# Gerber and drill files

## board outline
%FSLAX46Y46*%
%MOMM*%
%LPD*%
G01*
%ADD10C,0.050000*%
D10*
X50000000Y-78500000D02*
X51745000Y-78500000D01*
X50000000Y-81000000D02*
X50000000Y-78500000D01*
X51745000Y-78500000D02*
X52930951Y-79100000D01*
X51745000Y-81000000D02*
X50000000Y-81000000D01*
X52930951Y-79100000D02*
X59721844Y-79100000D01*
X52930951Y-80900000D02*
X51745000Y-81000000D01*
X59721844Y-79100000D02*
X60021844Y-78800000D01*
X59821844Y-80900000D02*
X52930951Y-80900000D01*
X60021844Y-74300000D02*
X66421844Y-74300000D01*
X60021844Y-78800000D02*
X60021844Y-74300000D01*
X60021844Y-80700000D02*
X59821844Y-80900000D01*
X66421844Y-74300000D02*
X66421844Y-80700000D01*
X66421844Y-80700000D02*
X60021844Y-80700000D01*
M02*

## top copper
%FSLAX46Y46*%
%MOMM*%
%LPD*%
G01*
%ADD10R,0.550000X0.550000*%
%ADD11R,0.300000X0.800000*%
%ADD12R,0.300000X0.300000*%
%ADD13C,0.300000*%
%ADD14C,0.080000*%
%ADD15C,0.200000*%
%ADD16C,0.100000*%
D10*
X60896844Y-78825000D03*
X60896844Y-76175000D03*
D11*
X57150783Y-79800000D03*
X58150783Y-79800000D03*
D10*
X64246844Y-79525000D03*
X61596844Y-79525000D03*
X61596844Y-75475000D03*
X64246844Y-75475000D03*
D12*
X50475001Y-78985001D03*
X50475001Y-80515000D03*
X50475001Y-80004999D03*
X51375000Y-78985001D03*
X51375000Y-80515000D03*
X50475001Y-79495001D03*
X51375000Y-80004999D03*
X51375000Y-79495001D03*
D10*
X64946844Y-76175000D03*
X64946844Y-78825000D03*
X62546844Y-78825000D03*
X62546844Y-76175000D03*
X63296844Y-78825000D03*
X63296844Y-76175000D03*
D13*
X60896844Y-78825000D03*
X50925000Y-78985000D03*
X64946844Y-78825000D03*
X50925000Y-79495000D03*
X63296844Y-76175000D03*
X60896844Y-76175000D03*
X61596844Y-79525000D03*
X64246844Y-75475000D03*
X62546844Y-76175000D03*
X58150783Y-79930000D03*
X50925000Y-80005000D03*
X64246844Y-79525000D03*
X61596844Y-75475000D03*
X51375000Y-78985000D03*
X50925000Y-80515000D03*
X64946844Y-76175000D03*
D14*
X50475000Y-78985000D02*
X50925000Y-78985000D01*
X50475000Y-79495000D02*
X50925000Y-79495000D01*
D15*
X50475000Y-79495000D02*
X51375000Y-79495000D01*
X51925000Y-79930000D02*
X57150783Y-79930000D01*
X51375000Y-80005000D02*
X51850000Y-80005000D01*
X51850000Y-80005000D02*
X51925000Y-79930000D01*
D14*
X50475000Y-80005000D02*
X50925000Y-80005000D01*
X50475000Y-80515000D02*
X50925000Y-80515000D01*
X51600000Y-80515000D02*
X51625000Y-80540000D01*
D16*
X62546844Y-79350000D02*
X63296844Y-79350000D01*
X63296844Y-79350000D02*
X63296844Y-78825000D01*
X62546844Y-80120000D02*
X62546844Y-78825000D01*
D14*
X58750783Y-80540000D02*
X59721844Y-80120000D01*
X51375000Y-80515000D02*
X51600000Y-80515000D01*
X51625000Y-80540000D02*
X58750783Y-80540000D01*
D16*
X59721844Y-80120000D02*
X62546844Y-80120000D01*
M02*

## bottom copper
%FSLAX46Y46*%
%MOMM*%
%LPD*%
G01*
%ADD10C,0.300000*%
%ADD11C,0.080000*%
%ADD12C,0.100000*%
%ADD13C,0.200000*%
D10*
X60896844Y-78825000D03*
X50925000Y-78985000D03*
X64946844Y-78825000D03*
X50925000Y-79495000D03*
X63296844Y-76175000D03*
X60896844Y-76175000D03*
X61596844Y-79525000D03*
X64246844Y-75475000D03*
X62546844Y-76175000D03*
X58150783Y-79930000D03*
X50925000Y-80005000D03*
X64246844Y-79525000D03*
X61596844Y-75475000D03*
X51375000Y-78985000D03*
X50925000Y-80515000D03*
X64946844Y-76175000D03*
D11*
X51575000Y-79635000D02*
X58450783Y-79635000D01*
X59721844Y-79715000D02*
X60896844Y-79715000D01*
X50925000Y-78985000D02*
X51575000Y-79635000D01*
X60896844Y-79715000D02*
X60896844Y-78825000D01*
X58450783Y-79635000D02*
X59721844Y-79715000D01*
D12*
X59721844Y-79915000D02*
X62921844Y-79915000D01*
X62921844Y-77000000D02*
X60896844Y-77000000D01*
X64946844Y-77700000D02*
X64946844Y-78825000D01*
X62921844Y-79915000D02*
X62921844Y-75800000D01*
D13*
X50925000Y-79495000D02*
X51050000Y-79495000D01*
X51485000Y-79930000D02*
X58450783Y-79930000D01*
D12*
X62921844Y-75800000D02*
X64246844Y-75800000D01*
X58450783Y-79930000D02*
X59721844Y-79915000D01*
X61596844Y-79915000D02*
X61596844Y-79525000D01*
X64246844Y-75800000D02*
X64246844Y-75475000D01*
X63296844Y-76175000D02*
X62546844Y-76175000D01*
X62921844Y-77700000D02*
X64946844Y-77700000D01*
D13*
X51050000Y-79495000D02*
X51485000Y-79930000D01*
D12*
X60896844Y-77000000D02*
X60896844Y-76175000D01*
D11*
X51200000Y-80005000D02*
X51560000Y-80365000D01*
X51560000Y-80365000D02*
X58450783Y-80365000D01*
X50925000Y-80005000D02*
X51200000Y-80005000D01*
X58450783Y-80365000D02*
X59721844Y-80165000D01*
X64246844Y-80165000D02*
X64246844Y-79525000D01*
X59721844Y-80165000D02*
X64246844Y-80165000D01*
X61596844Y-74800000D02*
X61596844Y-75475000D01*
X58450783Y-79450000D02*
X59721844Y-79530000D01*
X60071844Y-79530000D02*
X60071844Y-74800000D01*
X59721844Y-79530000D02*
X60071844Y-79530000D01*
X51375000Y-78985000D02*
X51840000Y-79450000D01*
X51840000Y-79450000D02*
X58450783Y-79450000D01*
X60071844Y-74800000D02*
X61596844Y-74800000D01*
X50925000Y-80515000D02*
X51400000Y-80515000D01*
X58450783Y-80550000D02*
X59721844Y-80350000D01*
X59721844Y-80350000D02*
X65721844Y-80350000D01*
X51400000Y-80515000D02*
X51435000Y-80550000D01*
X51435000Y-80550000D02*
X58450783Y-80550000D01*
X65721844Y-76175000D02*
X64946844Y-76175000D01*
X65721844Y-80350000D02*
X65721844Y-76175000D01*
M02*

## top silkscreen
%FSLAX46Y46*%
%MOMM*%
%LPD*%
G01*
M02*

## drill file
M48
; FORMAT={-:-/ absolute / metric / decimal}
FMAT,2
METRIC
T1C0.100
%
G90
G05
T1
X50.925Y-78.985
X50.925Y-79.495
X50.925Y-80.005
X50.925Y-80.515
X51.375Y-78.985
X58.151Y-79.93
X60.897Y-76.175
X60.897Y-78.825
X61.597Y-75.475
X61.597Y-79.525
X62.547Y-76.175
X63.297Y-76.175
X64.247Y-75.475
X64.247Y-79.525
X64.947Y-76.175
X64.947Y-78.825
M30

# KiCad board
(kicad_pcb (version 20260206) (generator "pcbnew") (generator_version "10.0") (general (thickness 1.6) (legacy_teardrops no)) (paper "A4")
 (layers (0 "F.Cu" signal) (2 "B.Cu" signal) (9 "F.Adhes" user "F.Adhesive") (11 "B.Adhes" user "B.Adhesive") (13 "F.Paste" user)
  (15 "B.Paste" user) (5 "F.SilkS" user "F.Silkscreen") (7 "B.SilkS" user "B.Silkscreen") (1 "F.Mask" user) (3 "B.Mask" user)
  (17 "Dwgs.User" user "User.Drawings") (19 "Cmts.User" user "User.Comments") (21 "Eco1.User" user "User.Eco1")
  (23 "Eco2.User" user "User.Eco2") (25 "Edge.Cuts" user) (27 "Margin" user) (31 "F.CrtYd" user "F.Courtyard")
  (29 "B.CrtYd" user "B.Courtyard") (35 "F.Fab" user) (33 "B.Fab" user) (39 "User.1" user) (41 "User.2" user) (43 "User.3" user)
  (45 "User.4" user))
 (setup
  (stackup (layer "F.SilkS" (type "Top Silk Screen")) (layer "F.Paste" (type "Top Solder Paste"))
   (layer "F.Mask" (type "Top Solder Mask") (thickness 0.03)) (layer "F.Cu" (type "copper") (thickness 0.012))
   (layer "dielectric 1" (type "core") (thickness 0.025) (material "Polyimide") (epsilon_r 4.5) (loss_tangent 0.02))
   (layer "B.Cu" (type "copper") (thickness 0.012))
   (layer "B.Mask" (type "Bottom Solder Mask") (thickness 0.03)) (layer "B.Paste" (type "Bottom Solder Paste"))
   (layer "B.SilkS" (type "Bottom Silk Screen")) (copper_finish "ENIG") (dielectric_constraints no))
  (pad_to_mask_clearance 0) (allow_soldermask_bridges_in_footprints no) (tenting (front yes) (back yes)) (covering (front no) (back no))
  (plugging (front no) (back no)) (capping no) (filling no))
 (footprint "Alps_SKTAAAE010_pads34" (layer "F.Cu") (at 60.521844 77.5 90)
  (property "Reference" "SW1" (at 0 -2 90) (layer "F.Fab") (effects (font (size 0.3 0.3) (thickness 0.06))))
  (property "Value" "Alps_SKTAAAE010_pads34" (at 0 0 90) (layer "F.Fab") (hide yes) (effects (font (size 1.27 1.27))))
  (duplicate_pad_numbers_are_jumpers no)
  (pad "3" smd rect (at -1.325 0.375 90) (size 0.55 0.55) (layers "F.Cu" "F.Mask") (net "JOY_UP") (solder_mask_margin 0.05)
   (thermal_bridge_angle 45))
  (pad "4" smd rect (at 1.325 0.375 90) (size 0.55 0.55) (layers "F.Cu" "F.Mask") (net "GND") (solder_mask_margin 0.05)
   (thermal_bridge_angle 45)))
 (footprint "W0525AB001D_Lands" (layer "F.Cu") (at 57.650783 79.93)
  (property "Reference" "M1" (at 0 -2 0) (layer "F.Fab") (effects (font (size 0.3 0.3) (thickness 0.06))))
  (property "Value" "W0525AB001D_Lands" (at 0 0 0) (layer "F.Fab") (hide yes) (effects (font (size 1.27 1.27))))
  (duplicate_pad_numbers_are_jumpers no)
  (pad "1" smd rect (at -0.5 -0.13) (size 0.3 0.8) (layers "F.Cu" "F.Mask") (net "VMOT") (solder_mask_margin 0.05) (thermal_bridge_angle 45))
  (pad "2" smd rect (at 0.5 -0.13) (size 0.3 0.8) (layers "F.Cu" "F.Mask") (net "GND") (solder_mask_margin 0.05) (thermal_bridge_angle 45)))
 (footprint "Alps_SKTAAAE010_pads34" (layer "F.Cu") (at 62.921844 79.9 180)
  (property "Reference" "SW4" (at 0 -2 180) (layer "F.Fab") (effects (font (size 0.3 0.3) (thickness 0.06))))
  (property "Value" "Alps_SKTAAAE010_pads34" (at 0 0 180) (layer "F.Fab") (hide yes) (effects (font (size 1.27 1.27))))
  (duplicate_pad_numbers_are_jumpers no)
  (pad "3" smd rect (at -1.325 0.375 180) (size 0.55 0.55) (layers "F.Cu" "F.Mask") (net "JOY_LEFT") (solder_mask_margin 0.05)
   (thermal_bridge_angle 45))
  (pad "4" smd rect (at 1.325 0.375 180) (size 0.55 0.55) (layers "F.Cu" "F.Mask") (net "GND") (solder_mask_margin 0.05)
   (thermal_bridge_angle 45)))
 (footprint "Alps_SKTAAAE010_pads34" (layer "F.Cu") (at 62.921844 75.1)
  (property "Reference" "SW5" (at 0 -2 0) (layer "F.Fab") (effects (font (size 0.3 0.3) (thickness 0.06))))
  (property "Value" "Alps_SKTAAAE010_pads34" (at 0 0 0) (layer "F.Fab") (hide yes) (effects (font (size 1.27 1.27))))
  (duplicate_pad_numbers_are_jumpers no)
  (pad "3" smd rect (at -1.325 0.375) (size 0.55 0.55) (layers "F.Cu" "F.Mask") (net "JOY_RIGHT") (solder_mask_margin 0.05)
   (thermal_bridge_angle 45))
  (pad "4" smd rect (at 1.325 0.375) (size 0.55 0.55) (layers "F.Cu" "F.Mask") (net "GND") (solder_mask_margin 0.05)
   (thermal_bridge_angle 45)))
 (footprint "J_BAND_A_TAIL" (layer "F.Cu") (at 50.9 79.75)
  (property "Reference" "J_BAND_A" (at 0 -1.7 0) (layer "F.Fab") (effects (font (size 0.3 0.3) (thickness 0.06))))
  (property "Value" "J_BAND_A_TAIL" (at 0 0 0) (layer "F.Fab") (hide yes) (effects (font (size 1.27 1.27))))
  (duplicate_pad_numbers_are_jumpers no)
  (pad "1" smd rect (at -0.424999 -0.764999) (size 0.3 0.3) (layers "F.Cu" "F.Mask") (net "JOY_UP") (solder_mask_margin 0.05)
   (thermal_bridge_angle 45))
  (pad "2" smd rect (at -0.424999 0.765) (size 0.3 0.3) (layers "F.Cu" "F.Mask") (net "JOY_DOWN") (solder_mask_margin 0.05)
   (thermal_bridge_angle 45))
  (pad "3" smd rect (at -0.424999 0.254999) (size 0.3 0.3) (layers "F.Cu" "F.Mask") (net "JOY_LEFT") (solder_mask_margin 0.05)
   (thermal_bridge_angle 45))
  (pad "4" smd rect (at 0.475 -0.764999) (size 0.3 0.3) (layers "F.Cu" "F.Mask") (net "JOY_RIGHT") (solder_mask_margin 0.05)
   (thermal_bridge_angle 45))
  (pad "5" smd rect (at 0.475 0.765) (size 0.3 0.3) (layers "F.Cu" "F.Mask") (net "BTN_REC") (solder_mask_margin 0.05)
   (thermal_bridge_angle 45))
  (pad "6" smd rect (at -0.424999 -0.254999) (size 0.3 0.3) (layers "F.Cu" "F.Mask") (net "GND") (solder_mask_margin 0.05)
   (thermal_bridge_angle 45))
  (pad "7" smd rect (at 0.475 0.254999) (size 0.3 0.3) (layers "F.Cu" "F.Mask") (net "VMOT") (solder_mask_margin 0.05)
   (thermal_bridge_angle 45))
  (pad "8" smd rect (at 0.475 -0.254999) (size 0.3 0.3) (layers "F.Cu" "F.Mask") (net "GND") (solder_mask_margin 0.05)
   (thermal_bridge_angle 45)))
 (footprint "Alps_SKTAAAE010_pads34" (layer "F.Cu") (at 65.321844 77.5 -90)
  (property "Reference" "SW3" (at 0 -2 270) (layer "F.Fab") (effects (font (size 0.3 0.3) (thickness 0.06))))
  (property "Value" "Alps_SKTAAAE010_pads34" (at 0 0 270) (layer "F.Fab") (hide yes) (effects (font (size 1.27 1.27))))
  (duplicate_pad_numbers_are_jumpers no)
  (pad "3" smd rect (at -1.325 0.375 270) (size 0.55 0.55) (layers "F.Cu" "F.Mask") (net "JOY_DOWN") (solder_mask_margin 0.05)
   (thermal_bridge_angle 45))
  (pad "4" smd rect (at 1.325 0.375 270) (size 0.55 0.55) (layers "F.Cu" "F.Mask") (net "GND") (solder_mask_margin 0.05)
   (thermal_bridge_angle 45)))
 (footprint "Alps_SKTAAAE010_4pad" (layer "F.Cu") (at 62.921844 77.5 90)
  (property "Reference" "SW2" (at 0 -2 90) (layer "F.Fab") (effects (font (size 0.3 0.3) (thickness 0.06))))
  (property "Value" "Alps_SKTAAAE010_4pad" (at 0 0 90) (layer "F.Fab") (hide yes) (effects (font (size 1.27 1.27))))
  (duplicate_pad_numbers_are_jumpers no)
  (pad "1" smd rect (at -1.325 -0.375 90) (size 0.55 0.55) (layers "F.Cu" "F.Mask") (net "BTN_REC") (solder_mask_margin 0.05)
   (thermal_bridge_angle 45))
  (pad "2" smd rect (at 1.325 -0.375 90) (size 0.55 0.55) (layers "F.Cu" "F.Mask") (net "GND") (solder_mask_margin 0.05)
   (thermal_bridge_angle 45))
  (pad "3" smd rect (at -1.325 0.375 90) (size 0.55 0.55) (layers "F.Cu" "F.Mask") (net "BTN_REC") (solder_mask_margin 0.05)
   (thermal_bridge_angle 45))
  (pad "4" smd rect (at 1.325 0.375 90) (size 0.55 0.55) (layers "F.Cu" "F.Mask") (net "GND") (solder_mask_margin 0.05)
   (thermal_bridge_angle 45)))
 (gr_line (start 50 78.5) (end 51.745 78.5) (stroke (width 0.05) (type default)) (layer "Edge.Cuts"))
 (gr_line (start 50 81) (end 50 78.5) (stroke (width 0.05) (type default)) (layer "Edge.Cuts"))
 (gr_line (start 51.745 78.5) (end 52.930951 79.1) (stroke (width 0.05) (type default)) (layer "Edge.Cuts"))
 (gr_line (start 51.745 81) (end 50 81) (stroke (width 0.05) (type default)) (layer "Edge.Cuts"))
 (gr_line (start 52.930951 79.1) (end 59.721844 79.1) (stroke (width 0.05) (type default)) (layer "Edge.Cuts"))
 (gr_line (start 52.930951 80.9) (end 51.745 81) (stroke (width 0.05) (type default)) (layer "Edge.Cuts"))
 (gr_line (start 59.721844 79.1) (end 60.021844 78.8) (stroke (width 0.05) (type default)) (layer "Edge.Cuts"))
 (gr_line (start 59.821844 80.9) (end 52.930951 80.9) (stroke (width 0.05) (type default)) (layer "Edge.Cuts"))
 (gr_line (start 60.021844 74.3) (end 66.421844 74.3) (stroke (width 0.05) (type default)) (layer "Edge.Cuts"))
 (gr_line (start 60.021844 78.8) (end 60.021844 74.3) (stroke (width 0.05) (type default)) (layer "Edge.Cuts"))
 (gr_line (start 60.021844 80.7) (end 59.821844 80.9) (stroke (width 0.05) (type default)) (layer "Edge.Cuts"))
 (gr_line (start 66.421844 74.3) (end 66.421844 80.7) (stroke (width 0.05) (type default)) (layer "Edge.Cuts"))
 (gr_line (start 66.421844 80.7) (end 60.021844 80.7) (stroke (width 0.05) (type default)) (layer "Edge.Cuts"))
 (segment (start 50.475 78.985) (end 50.925 78.985) (width 0.08) (layer "F.Cu") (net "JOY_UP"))
 (via (at 60.896844 78.825) (size 0.3) (drill 0.1) (layers "F.Cu" "B.Cu") (tenting (front yes) (back yes)) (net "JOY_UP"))
 (via (at 50.925 78.985) (size 0.3) (drill 0.1) (layers "F.Cu" "B.Cu") (tenting (front yes) (back yes)) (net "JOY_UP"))
 (segment (start 51.575 79.635) (end 58.450783 79.635) (width 0.08) (layer "B.Cu") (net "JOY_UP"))
 (segment (start 59.721844 79.715) (end 60.896844 79.715) (width 0.08) (layer "B.Cu") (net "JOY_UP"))
 (segment (start 50.925 78.985) (end 51.575 79.635) (width 0.08) (layer "B.Cu") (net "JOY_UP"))
 (segment (start 60.896844 79.715) (end 60.896844 78.825) (width 0.08) (layer "B.Cu") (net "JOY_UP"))
 (segment (start 58.450783 79.635) (end 59.721844 79.715) (width 0.08) (layer "B.Cu") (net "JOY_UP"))
 (segment (start 50.475 79.495) (end 50.925 79.495) (width 0.08) (layer "F.Cu") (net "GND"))
 (segment (start 50.475 79.495) (end 51.375 79.495) (width 0.2) (layer "F.Cu") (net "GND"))
 (via (at 64.946844 78.825) (size 0.3) (drill 0.1) (layers "F.Cu" "B.Cu") (tenting (front yes) (back yes)) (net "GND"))
 (via (at 50.925 79.495) (size 0.3) (drill 0.1) (layers "F.Cu" "B.Cu") (tenting (front yes) (back yes)) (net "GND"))
 (via (at 63.296844 76.175) (size 0.3) (drill 0.1) (layers "F.Cu" "B.Cu") (tenting (front yes) (back yes)) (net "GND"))
 (via (at 60.896844 76.175) (size 0.3) (drill 0.1) (layers "F.Cu" "B.Cu") (tenting (front yes) (back yes)) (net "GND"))
 (via (at 61.596844 79.525) (size 0.3) (drill 0.1) (layers "F.Cu" "B.Cu") (tenting (front yes) (back yes)) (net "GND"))
 (via (at 64.246844 75.475) (size 0.3) (drill 0.1) (layers "F.Cu" "B.Cu") (tenting (front yes) (back yes)) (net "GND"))
 (via (at 62.546844 76.175) (size 0.3) (drill 0.1) (layers "F.Cu" "B.Cu") (tenting (front yes) (back yes)) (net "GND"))
 (via (at 58.150783 79.93) (size 0.3) (drill 0.1) (layers "F.Cu" "B.Cu") (tenting (front yes) (back yes)) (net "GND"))
 (segment (start 59.721844 79.915) (end 62.921844 79.915) (width 0.1) (layer "B.Cu") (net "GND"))
 (segment (start 62.921844 77) (end 60.896844 77) (width 0.1) (layer "B.Cu") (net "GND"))
 (segment (start 64.946844 77.7) (end 64.946844 78.825) (width 0.1) (layer "B.Cu") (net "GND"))
 (segment (start 62.921844 79.915) (end 62.921844 75.8) (width 0.1) (layer "B.Cu") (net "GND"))
 (segment (start 50.925 79.495) (end 51.05 79.495) (width 0.2) (layer "B.Cu") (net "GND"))
 (segment (start 51.485 79.93) (end 58.450783 79.93) (width 0.2) (layer "B.Cu") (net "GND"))
 (segment (start 62.921844 75.8) (end 64.246844 75.8) (width 0.1) (layer "B.Cu") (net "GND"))
 (segment (start 58.450783 79.93) (end 59.721844 79.915) (width 0.1) (layer "B.Cu") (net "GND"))
 (segment (start 61.596844 79.915) (end 61.596844 79.525) (width 0.1) (layer "B.Cu") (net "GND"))
 (segment (start 64.246844 75.8) (end 64.246844 75.475) (width 0.1) (layer "B.Cu") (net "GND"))
 (segment (start 63.296844 76.175) (end 62.546844 76.175) (width 0.1) (layer "B.Cu") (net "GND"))
 (segment (start 62.921844 77.7) (end 64.946844 77.7) (width 0.1) (layer "B.Cu") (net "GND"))
 (segment (start 51.05 79.495) (end 51.485 79.93) (width 0.2) (layer "B.Cu") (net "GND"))
 (segment (start 60.896844 77) (end 60.896844 76.175) (width 0.1) (layer "B.Cu") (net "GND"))
 (segment (start 51.925 79.93) (end 57.150783 79.93) (width 0.2) (layer "F.Cu") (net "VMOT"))
 (segment (start 51.375 80.005) (end 51.85 80.005) (width 0.2) (layer "F.Cu") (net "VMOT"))
 (segment (start 51.85 80.005) (end 51.925 79.93) (width 0.2) (layer "F.Cu") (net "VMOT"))
 (segment (start 50.475 80.005) (end 50.925 80.005) (width 0.08) (layer "F.Cu") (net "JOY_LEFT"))
 (via (at 50.925 80.005) (size 0.3) (drill 0.1) (layers "F.Cu" "B.Cu") (tenting (front yes) (back yes)) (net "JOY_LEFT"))
 (via (at 64.246844 79.525) (size 0.3) (drill 0.1) (layers "F.Cu" "B.Cu") (tenting (front yes) (back yes)) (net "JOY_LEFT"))
 (segment (start 51.2 80.005) (end 51.56 80.365) (width 0.08) (layer "B.Cu") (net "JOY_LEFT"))
 (segment (start 51.56 80.365) (end 58.450783 80.365) (width 0.08) (layer "B.Cu") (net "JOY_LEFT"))
 (segment (start 50.925 80.005) (end 51.2 80.005) (width 0.08) (layer "B.Cu") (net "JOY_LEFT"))
 (segment (start 58.450783 80.365) (end 59.721844 80.165) (width 0.08) (layer "B.Cu") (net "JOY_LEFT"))
 (segment (start 64.246844 80.165) (end 64.246844 79.525) (width 0.08) (layer "B.Cu") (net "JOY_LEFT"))
 (segment (start 59.721844 80.165) (end 64.246844 80.165) (width 0.08) (layer "B.Cu") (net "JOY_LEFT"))
 (via (at 61.596844 75.475) (size 0.3) (drill 0.1) (layers "F.Cu" "B.Cu") (tenting (front yes) (back yes)) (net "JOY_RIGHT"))
 (via (at 51.375 78.985) (size 0.3) (drill 0.1) (layers "F.Cu" "B.Cu") (tenting (front yes) (back yes)) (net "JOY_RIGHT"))
 (segment (start 61.596844 74.8) (end 61.596844 75.475) (width 0.08) (layer "B.Cu") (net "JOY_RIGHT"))
 (segment (start 58.450783 79.45) (end 59.721844 79.53) (width 0.08) (layer "B.Cu") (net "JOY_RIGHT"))
 (segment (start 60.071844 79.53) (end 60.071844 74.8) (width 0.08) (layer "B.Cu") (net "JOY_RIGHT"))
 (segment (start 59.721844 79.53) (end 60.071844 79.53) (width 0.08) (layer "B.Cu") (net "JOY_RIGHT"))
 (segment (start 51.375 78.985) (end 51.84 79.45) (width 0.08) (layer "B.Cu") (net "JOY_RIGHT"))
 (segment (start 51.84 79.45) (end 58.450783 79.45) (width 0.08) (layer "B.Cu") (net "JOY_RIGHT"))
 (segment (start 60.071844 74.8) (end 61.596844 74.8) (width 0.08) (layer "B.Cu") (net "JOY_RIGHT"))
 (segment (start 50.475 80.515) (end 50.925 80.515) (width 0.08) (layer "F.Cu") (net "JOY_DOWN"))
 (via (at 50.925 80.515) (size 0.3) (drill 0.1) (layers "F.Cu" "B.Cu") (tenting (front yes) (back yes)) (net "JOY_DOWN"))
 (via (at 64.946844 76.175) (size 0.3) (drill 0.1) (layers "F.Cu" "B.Cu") (tenting (front yes) (back yes)) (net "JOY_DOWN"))
 (segment (start 50.925 80.515) (end 51.4 80.515) (width 0.08) (layer "B.Cu") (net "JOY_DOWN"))
 (segment (start 58.450783 80.55) (end 59.721844 80.35) (width 0.08) (layer "B.Cu") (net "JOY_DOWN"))
 (segment (start 59.721844 80.35) (end 65.721844 80.35) (width 0.08) (layer "B.Cu") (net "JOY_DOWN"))
 (segment (start 51.4 80.515) (end 51.435 80.55) (width 0.08) (layer "B.Cu") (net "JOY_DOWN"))
 (segment (start 51.435 80.55) (end 58.450783 80.55) (width 0.08) (layer "B.Cu") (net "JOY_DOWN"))
 (segment (start 65.721844 76.175) (end 64.946844 76.175) (width 0.08) (layer "B.Cu") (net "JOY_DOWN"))
 (segment (start 65.721844 80.35) (end 65.721844 76.175) (width 0.08) (layer "B.Cu") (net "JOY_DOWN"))
 (segment (start 51.6 80.515) (end 51.625 80.54) (width 0.08) (layer "F.Cu") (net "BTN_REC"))
 (segment (start 62.546844 79.35) (end 63.296844 79.35) (width 0.1) (layer "F.Cu") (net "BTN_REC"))
 (segment (start 63.296844 79.35) (end 63.296844 78.825) (width 0.1) (layer "F.Cu") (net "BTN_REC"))
 (segment (start 62.546844 80.12) (end 62.546844 78.825) (width 0.1) (layer "F.Cu") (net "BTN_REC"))
 (segment (start 58.750783 80.54) (end 59.721844 80.12) (width 0.08) (layer "F.Cu") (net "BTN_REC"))
 (segment (start 51.375 80.515) (end 51.6 80.515) (width 0.08) (layer "F.Cu") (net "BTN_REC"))
 (segment (start 51.625 80.54) (end 58.750783 80.54) (width 0.08) (layer "F.Cu") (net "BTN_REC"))
 (segment (start 59.721844 80.12) (end 62.546844 80.12) (width 0.1) (layer "F.Cu") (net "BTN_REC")))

